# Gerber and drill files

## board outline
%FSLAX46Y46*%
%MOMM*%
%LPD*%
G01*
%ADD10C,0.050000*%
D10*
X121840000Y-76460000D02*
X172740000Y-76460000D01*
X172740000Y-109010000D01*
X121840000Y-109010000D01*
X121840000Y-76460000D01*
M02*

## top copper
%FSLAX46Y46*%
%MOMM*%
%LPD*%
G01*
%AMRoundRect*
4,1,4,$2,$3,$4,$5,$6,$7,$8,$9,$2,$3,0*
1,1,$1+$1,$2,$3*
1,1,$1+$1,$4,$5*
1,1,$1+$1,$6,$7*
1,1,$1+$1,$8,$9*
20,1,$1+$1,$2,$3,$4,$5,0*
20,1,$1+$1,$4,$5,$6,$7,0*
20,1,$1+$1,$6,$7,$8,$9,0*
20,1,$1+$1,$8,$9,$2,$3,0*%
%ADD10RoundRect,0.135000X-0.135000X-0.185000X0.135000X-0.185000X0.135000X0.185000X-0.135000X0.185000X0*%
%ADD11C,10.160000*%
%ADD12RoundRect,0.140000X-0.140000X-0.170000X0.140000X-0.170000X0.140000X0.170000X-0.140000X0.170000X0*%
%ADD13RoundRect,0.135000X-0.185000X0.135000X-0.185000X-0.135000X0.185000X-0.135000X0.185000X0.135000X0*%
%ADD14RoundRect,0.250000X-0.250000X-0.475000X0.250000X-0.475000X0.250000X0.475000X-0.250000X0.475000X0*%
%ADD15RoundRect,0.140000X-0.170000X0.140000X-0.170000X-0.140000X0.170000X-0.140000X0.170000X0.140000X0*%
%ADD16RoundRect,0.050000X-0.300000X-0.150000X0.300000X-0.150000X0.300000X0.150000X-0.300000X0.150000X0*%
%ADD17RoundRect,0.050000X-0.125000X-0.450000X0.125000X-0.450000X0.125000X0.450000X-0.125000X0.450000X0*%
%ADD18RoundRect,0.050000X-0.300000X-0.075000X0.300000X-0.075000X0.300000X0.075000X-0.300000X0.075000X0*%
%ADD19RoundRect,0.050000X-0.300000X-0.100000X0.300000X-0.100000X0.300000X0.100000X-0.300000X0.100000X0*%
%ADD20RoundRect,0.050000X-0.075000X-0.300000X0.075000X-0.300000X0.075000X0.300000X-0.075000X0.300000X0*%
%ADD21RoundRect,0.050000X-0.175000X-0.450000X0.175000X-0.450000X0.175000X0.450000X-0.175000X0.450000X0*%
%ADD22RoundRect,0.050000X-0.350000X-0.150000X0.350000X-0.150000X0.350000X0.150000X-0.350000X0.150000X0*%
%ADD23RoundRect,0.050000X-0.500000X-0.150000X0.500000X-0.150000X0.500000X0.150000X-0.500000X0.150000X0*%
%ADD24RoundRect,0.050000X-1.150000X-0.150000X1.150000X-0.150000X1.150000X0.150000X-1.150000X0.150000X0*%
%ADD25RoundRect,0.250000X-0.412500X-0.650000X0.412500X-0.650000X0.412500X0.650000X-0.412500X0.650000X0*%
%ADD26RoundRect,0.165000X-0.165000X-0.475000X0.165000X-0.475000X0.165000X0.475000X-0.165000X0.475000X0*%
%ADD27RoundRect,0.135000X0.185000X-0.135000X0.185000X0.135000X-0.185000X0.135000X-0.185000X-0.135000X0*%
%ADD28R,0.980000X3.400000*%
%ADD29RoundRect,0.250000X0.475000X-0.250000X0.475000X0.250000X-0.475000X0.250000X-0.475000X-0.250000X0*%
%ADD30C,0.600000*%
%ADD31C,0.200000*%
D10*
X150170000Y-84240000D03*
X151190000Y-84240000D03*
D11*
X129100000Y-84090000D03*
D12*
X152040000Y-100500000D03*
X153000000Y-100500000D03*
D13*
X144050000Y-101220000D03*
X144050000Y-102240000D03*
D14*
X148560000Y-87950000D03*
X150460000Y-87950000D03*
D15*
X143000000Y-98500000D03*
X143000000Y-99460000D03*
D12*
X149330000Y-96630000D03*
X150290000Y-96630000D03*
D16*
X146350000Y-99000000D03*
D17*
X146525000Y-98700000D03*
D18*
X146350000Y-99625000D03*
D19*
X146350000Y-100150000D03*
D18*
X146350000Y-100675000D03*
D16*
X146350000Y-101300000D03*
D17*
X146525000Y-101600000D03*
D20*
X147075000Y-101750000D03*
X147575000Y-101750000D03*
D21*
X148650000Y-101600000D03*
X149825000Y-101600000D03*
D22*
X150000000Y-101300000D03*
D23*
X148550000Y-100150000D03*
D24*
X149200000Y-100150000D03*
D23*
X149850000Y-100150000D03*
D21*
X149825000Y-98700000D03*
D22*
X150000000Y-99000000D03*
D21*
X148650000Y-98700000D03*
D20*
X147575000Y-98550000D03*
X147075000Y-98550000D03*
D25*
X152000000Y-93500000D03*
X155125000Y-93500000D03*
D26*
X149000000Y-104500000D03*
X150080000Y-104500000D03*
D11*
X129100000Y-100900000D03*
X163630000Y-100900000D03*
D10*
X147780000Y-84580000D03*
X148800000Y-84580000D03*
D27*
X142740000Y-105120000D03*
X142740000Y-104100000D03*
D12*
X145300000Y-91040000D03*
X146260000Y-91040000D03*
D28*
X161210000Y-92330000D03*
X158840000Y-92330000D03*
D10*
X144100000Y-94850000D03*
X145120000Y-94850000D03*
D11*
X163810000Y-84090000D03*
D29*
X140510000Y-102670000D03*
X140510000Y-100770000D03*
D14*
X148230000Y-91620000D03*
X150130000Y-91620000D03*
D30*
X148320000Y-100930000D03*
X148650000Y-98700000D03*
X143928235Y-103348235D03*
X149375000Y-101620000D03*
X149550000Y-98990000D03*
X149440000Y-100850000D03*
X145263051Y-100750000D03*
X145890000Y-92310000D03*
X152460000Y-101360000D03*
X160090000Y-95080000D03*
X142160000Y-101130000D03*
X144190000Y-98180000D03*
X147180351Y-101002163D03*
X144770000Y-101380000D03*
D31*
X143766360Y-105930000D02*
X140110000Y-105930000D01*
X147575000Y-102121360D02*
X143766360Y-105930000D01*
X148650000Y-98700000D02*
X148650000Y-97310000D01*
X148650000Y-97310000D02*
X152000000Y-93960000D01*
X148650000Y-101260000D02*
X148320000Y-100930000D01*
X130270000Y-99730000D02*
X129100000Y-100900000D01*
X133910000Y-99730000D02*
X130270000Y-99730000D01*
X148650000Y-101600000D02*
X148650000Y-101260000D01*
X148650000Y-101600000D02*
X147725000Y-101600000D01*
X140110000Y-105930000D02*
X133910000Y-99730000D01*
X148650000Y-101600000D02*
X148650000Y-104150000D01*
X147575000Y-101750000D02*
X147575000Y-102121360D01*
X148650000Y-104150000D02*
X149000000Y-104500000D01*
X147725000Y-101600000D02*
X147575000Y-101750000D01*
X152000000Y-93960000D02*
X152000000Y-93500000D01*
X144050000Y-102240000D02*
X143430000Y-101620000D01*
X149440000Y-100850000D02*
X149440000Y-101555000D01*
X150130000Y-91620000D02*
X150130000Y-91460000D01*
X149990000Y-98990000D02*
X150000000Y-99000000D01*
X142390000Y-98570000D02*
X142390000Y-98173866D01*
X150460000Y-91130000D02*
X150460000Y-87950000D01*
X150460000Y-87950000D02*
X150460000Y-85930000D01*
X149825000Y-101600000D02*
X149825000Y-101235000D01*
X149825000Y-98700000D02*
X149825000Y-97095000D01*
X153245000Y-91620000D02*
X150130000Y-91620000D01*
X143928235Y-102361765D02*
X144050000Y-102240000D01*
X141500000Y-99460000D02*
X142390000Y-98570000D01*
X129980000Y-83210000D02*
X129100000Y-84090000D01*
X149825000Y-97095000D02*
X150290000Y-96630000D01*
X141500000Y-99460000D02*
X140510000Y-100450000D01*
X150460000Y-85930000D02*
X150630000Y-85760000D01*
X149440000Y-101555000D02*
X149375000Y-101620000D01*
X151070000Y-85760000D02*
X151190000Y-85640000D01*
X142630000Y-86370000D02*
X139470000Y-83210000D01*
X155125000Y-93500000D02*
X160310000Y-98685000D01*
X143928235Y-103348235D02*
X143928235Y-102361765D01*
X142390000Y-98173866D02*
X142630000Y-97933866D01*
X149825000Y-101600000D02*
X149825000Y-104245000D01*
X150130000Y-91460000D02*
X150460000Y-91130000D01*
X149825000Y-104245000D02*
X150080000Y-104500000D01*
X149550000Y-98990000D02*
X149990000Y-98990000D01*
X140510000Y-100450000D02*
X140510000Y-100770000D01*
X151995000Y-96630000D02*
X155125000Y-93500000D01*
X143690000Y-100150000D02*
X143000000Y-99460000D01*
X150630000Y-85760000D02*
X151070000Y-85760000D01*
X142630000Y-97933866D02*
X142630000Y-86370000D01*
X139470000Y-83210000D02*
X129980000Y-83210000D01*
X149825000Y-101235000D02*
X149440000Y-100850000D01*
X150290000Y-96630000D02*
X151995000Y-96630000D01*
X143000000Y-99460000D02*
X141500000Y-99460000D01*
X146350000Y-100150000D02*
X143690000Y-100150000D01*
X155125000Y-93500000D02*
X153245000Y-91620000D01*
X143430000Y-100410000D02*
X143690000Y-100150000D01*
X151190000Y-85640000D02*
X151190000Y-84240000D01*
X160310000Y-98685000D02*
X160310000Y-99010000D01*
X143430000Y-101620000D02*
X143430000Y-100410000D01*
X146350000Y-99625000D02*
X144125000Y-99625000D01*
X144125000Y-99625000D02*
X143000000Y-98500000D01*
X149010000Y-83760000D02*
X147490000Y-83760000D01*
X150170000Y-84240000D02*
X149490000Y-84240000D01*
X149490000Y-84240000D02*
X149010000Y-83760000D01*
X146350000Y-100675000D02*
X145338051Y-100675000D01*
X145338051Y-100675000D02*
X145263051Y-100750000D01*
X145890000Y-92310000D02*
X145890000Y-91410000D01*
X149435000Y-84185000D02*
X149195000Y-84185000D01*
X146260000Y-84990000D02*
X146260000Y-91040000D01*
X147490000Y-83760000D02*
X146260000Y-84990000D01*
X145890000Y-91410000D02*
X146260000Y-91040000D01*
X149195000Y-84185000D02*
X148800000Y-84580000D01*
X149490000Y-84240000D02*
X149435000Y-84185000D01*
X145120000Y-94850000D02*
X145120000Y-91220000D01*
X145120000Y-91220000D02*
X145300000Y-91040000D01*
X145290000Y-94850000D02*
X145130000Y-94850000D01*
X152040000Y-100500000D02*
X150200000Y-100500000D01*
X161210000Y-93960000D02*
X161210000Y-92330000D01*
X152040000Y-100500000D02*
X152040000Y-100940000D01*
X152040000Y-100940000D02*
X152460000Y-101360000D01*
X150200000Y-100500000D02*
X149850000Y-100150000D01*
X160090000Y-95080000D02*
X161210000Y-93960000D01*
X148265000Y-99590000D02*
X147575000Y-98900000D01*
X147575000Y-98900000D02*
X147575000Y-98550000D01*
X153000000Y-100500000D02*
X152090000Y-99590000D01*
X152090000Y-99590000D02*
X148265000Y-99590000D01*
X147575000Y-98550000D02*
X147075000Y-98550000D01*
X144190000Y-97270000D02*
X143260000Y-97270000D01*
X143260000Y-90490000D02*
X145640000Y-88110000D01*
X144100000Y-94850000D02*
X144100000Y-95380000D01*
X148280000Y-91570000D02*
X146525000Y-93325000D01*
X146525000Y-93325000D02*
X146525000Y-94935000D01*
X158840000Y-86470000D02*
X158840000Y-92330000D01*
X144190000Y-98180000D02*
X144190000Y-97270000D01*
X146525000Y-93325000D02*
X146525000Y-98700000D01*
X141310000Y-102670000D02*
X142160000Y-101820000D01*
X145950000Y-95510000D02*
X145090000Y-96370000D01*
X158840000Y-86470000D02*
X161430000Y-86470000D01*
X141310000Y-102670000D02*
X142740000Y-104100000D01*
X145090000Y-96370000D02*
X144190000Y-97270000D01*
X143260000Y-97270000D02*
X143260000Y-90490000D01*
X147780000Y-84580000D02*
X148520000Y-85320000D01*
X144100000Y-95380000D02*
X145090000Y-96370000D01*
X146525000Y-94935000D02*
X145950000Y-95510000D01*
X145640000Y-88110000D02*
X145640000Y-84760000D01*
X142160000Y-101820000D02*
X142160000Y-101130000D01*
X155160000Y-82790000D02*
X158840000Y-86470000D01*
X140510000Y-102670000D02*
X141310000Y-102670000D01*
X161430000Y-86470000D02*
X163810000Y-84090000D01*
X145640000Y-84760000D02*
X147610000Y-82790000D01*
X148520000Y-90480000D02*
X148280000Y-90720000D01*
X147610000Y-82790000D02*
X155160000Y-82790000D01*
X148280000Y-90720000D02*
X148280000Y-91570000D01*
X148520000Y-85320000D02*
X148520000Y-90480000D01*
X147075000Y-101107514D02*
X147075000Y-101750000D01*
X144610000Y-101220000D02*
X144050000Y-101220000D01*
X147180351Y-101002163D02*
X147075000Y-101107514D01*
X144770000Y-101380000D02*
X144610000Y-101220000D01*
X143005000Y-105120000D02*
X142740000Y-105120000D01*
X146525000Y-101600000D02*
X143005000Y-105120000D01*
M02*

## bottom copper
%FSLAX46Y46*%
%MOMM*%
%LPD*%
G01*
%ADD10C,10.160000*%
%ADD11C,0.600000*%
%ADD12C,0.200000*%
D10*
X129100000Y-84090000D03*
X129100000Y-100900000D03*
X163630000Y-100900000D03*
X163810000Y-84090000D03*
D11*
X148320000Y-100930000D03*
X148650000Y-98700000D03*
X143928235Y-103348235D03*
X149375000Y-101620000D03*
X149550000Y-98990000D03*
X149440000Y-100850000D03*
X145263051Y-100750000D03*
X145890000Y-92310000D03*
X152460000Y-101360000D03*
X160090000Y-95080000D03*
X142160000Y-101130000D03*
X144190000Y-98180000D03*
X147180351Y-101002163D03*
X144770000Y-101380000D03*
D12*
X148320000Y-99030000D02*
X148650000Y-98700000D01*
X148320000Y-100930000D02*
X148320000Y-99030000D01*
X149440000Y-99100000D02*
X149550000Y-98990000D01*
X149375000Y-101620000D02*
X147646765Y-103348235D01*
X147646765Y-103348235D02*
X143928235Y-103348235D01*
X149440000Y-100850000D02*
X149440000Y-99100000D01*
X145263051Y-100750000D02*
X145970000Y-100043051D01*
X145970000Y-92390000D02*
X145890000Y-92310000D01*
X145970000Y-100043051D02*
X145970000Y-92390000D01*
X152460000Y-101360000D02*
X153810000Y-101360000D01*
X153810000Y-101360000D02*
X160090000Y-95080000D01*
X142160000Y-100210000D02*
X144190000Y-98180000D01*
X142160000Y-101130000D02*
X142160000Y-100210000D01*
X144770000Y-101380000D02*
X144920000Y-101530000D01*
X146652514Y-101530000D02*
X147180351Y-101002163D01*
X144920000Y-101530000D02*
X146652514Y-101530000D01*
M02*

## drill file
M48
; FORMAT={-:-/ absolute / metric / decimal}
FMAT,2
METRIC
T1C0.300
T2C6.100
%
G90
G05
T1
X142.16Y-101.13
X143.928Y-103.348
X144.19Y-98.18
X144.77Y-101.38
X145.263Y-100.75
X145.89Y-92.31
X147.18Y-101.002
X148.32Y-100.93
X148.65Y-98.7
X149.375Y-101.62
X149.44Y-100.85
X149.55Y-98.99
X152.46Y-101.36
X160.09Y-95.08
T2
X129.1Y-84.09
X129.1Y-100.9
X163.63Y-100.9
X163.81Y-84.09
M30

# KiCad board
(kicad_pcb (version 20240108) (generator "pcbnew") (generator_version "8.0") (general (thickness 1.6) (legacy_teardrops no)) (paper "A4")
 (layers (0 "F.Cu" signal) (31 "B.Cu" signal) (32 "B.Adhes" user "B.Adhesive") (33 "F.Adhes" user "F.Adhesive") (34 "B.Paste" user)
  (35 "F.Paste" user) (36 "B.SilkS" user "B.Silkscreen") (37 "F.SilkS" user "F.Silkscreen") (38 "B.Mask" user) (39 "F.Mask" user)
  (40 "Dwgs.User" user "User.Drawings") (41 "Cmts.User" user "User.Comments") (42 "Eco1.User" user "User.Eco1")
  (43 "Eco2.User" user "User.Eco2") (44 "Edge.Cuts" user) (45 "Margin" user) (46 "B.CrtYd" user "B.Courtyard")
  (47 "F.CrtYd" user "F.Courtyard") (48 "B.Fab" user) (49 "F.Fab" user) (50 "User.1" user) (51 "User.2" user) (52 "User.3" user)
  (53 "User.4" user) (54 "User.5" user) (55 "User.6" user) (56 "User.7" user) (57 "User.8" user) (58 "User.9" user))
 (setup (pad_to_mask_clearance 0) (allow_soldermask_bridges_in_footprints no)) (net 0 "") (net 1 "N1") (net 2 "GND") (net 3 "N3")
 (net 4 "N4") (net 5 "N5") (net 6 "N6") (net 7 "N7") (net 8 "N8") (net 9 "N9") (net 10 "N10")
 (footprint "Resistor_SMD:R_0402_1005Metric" (layer "F.Cu") (at 150.68 84.24)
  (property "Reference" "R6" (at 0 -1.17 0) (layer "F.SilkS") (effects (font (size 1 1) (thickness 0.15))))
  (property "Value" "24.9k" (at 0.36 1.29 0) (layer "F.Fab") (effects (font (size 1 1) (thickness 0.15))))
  (pad "1" smd roundrect (at -0.51 0) (size 0.54 0.64) (layers "F.Cu" "F.Paste" "F.Mask") (roundrect_rratio 0.25) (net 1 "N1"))
  (pad "2" smd roundrect (at 0.51 0) (size 0.54 0.64) (layers "F.Cu" "F.Paste" "F.Mask") (roundrect_rratio 0.25) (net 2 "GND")))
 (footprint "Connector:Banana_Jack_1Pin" (layer "F.Cu") (at 129.1 84.09)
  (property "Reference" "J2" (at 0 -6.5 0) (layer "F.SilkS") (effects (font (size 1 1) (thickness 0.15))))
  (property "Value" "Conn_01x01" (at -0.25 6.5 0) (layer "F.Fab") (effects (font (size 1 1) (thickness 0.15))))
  (pad "1" thru_hole circle (at 0 0) (size 10.16 10.16) (drill 6.1) (layers "*.Cu" "*.Mask") (remove_unused_layers no) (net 2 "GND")))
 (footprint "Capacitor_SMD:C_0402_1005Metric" (layer "F.Cu") (at 152.52 100.5)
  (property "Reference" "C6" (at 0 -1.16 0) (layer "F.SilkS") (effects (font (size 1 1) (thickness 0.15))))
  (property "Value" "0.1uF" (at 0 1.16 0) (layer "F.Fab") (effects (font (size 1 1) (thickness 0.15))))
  (pad "1" smd roundrect (at -0.48 0) (size 0.56 0.62) (layers "F.Cu" "F.Paste" "F.Mask") (roundrect_rratio 0.25) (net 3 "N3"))
  (pad "2" smd roundrect (at 0.48 0) (size 0.56 0.62) (layers "F.Cu" "F.Paste" "F.Mask") (roundrect_rratio 0.25) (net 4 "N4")))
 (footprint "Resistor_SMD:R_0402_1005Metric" (layer "F.Cu") (at 144.05 101.73 -90)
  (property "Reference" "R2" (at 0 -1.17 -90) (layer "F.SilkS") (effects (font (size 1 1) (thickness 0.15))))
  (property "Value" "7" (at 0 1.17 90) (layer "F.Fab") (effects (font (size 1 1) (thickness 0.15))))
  (pad "1" smd roundrect (at -0.51 0 270) (size 0.54 0.64) (layers "F.Cu" "F.Paste" "F.Mask") (roundrect_rratio 0.25) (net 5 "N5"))
  (pad "2" smd roundrect (at 0.51 0 270) (size 0.54 0.64) (layers "F.Cu" "F.Paste" "F.Mask") (roundrect_rratio 0.25) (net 2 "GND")))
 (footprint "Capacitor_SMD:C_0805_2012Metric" (layer "F.Cu") (at 149.51 87.95)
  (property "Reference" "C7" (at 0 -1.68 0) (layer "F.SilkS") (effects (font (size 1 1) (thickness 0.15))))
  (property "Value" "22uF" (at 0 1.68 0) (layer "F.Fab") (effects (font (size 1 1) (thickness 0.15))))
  (pad "1" smd roundrect (at -0.95 0) (size 1 1.45) (layers "F.Cu" "F.Paste" "F.Mask") (roundrect_rratio 0.25) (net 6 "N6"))
  (pad "2" smd roundrect (at 0.95 0) (size 1 1.45) (layers "F.Cu" "F.Paste" "F.Mask") (roundrect_rratio 0.25) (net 2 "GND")))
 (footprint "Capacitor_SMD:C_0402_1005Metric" (layer "F.Cu") (at 143 98.98 -90)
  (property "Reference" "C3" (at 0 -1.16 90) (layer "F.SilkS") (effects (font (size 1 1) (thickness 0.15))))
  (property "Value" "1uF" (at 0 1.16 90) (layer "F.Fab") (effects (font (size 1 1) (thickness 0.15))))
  (pad "1" smd roundrect (at -0.48 0 270) (size 0.56 0.62) (layers "F.Cu" "F.Paste" "F.Mask") (roundrect_rratio 0.25) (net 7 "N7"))
  (pad "2" smd roundrect (at 0.48 0 270) (size 0.56 0.62) (layers "F.Cu" "F.Paste" "F.Mask") (roundrect_rratio 0.25) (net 2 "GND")))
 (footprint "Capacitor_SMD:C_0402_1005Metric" (layer "F.Cu") (at 149.81 96.63)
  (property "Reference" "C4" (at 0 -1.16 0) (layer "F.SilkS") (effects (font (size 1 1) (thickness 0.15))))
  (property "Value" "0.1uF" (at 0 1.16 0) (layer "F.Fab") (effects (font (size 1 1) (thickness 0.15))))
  (pad "1" smd roundrect (at -0.48 0) (size 0.56 0.62) (layers "F.Cu" "F.Paste" "F.Mask") (roundrect_rratio 0.25) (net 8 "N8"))
  (pad "2" smd roundrect (at 0.48 0) (size 0.56 0.62) (layers "F.Cu" "F.Paste" "F.Mask") (roundrect_rratio 0.25) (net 2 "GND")))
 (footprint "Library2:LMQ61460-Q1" (layer "F.Cu") (at 148.2 100.15)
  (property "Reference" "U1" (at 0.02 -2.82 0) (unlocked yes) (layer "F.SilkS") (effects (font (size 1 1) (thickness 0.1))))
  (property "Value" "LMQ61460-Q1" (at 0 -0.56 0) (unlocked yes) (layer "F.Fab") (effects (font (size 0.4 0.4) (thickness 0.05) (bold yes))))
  (pad "1" smd roundrect (at -1.85 -1.15) (size 0.7 0.4) (layers "F.Cu" "F.Paste" "F.Mask") (roundrect_rratio 0.125) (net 6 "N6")
   (solder_paste_margin_ratio -0.05) (thermal_bridge_angle 45))
  (pad "1" smd roundrect (at -1.675 -1.45) (size 0.35 1) (layers "F.Cu" "F.Paste" "F.Mask") (roundrect_rratio 0.1428571429) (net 6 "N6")
   (solder_paste_margin_ratio -0.05) (thermal_bridge_angle 45))
  (pad "2" smd roundrect (at -1.85 -0.525) (size 0.7 0.25) (layers "F.Cu" "F.Paste" "F.Mask") (roundrect_rratio 0.2) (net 7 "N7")
   (thermal_bridge_angle 45))
  (pad "3" smd roundrect (at -1.85 0) (size 0.7 0.3) (layers "F.Cu" "F.Paste" "F.Mask") (roundrect_rratio 0.1666666667) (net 2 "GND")
   (thermal_bridge_angle 45))
  (pad "4" smd roundrect (at -1.85 0.525) (size 0.7 0.25) (layers "F.Cu" "F.Paste" "F.Mask") (roundrect_rratio 0.2) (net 1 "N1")
   (thermal_bridge_angle 45))
  (pad "5" smd roundrect (at -1.85 1.15) (size 0.7 0.4) (layers "F.Cu" "F.Paste" "F.Mask") (roundrect_rratio 0.125) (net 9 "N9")
   (solder_paste_margin_ratio -0.05) (thermal_bridge_angle 45))
  (pad "5" smd roundrect (at -1.675 1.45) (size 0.35 1) (layers "F.Cu" "F.Paste" "F.Mask") (roundrect_rratio 0.1428571429) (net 9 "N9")
   (solder_paste_margin_ratio -0.05) (thermal_bridge_angle 45))
  (pad "6" smd roundrect (at -1.125 1.6) (size 0.25 0.7) (layers "F.Cu" "F.Paste" "F.Mask") (roundrect_rratio 0.2) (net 5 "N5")
   (thermal_bridge_angle 45))
  (pad "7" smd roundrect (at -0.625 1.6) (size 0.25 0.7) (layers "F.Cu" "F.Paste" "F.Mask") (roundrect_rratio 0.2) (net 8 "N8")
   (thermal_bridge_angle 45))
  (pad "8" smd roundrect (at 0.45 1.45) (size 0.45 1) (layers "F.Cu" "F.Paste" "F.Mask") (roundrect_rratio 0.1111111111) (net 8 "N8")
   (thermal_bridge_angle 45))
  (pad "9" smd roundrect (at 1.625 1.45) (size 0.45 1) (layers "F.Cu" "F.Paste" "F.Mask") (roundrect_rratio 0.1111111111) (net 2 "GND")
   (solder_paste_margin_ratio -0.05) (thermal_bridge_angle 45))
  (pad "9" smd roundrect (at 1.8 1.15) (size 0.8 0.4) (layers "F.Cu" "F.Paste" "F.Mask") (roundrect_rratio 0.125) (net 2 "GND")
   (solder_paste_margin_ratio -0.05) (thermal_bridge_angle 45))
  (pad "10" smd roundrect (at 0.35 0) (size 1.1 0.4) (layers "F.Cu" "F.Paste" "F.Mask") (roundrect_rratio 0.125) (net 3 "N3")
   (thermal_bridge_angle 45))
  (pad "10" smd roundrect (at 1 0) (size 2.4 0.4) (layers "F.Cu" "F.Paste" "F.Mask") (roundrect_rratio 0.125) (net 3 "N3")
   (thermal_bridge_angle 45))
  (pad "10" smd roundrect (at 1.65 0) (size 1.1 0.4) (layers "F.Cu" "F.Paste" "F.Mask") (roundrect_rratio 0.125) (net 3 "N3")
   (thermal_bridge_angle 45))
  (pad "11" smd roundrect (at 1.625 -1.45) (size 0.45 1) (layers "F.Cu" "F.Paste" "F.Mask") (roundrect_rratio 0.1111111111) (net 2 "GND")
   (solder_paste_margin_ratio -0.05) (thermal_bridge_angle 45))
  (pad "11" smd roundrect (at 1.8 -1.15) (size 0.8 0.4) (layers "F.Cu" "F.Paste" "F.Mask") (roundrect_rratio 0.125) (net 2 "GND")
   (solder_paste_margin_ratio -0.05) (thermal_bridge_angle 45))
  (pad "12" smd roundrect (at 0.45 -1.45) (size 0.45 1) (layers "F.Cu" "F.Paste" "F.Mask") (roundrect_rratio 0.1111111111) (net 8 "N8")
   (thermal_bridge_angle 45))
  (pad "13" smd roundrect (at -0.625 -1.6) (size 0.25 0.7) (layers "F.Cu" "F.Paste" "F.Mask") (roundrect_rratio 0.2) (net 4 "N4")
   (thermal_bridge_angle 45))
  (pad "14" smd roundrect (at -1.125 -1.6) (size 0.25 0.7) (layers "F.Cu" "F.Paste" "F.Mask") (roundrect_rratio 0.2) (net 4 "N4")
   (thermal_bridge_angle 45)))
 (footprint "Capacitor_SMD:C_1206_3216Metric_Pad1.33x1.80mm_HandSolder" (layer "F.Cu") (at 153.5625 93.5)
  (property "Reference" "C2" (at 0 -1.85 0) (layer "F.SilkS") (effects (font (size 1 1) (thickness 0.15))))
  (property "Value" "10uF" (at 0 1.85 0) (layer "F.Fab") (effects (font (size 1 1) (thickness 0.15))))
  (pad "1" smd roundrect (at -1.5625 0) (size 1.325 1.8) (layers "F.Cu" "F.Paste" "F.Mask") (roundrect_rratio 0.188679) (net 8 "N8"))
  (pad "2" smd roundrect (at 1.5625 0) (size 1.325 1.8) (layers "F.Cu" "F.Paste" "F.Mask") (roundrect_rratio 0.188679) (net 2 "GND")))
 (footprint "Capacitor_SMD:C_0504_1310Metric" (layer "F.Cu") (at 149.54 104.5)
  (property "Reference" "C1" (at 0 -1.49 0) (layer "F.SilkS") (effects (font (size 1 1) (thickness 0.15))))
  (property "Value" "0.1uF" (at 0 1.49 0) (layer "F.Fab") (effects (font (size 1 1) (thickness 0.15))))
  (pad "1" smd roundrect (at -0.54 0) (size 0.66 1.28) (layers "F.Cu" "F.Paste" "F.Mask") (roundrect_rratio 0.25) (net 8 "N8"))
  (pad "2" smd roundrect (at 0.54 0) (size 0.66 1.28) (layers "F.Cu" "F.Paste" "F.Mask") (roundrect_rratio 0.25) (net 2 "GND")))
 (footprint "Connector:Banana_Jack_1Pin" (layer "F.Cu") (at 129.1 100.9)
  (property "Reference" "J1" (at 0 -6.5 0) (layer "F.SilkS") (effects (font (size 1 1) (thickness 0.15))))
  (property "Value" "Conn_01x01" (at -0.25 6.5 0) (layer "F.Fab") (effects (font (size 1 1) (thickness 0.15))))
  (pad "1" thru_hole circle (at 0 0) (size 10.16 10.16) (drill 6.1) (layers "*.Cu" "*.Mask") (remove_unused_layers no) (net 8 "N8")))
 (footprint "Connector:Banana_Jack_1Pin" (layer "F.Cu") (at 163.63 100.9)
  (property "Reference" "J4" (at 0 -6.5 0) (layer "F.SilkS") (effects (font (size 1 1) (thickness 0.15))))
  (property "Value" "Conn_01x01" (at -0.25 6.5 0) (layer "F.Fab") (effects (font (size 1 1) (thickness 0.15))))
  (pad "1" thru_hole circle (at 0 0) (size 10.16 10.16) (drill 6.1) (layers "*.Cu" "*.Mask") (remove_unused_layers no) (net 2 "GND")))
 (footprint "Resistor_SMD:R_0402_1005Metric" (layer "F.Cu") (at 148.29 84.58)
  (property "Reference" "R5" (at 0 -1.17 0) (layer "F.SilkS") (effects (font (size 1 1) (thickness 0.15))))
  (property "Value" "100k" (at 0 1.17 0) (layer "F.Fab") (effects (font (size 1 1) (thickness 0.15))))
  (pad "1" smd roundrect (at -0.51 0) (size 0.54 0.64) (layers "F.Cu" "F.Paste" "F.Mask") (roundrect_rratio 0.25) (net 6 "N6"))
  (pad "2" smd roundrect (at 0.51 0) (size 0.54 0.64) (layers "F.Cu" "F.Paste" "F.Mask") (roundrect_rratio 0.25) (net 1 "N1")))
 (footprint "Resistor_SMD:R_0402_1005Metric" (layer "F.Cu") (at 142.74 104.61 90)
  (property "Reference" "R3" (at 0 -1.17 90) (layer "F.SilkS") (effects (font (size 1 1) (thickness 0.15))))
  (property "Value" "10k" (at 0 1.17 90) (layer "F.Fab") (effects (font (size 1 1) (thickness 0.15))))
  (pad "1" smd roundrect (at -0.51 0 90) (size 0.54 0.64) (layers "F.Cu" "F.Paste" "F.Mask") (roundrect_rratio 0.25) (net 9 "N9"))
  (pad "2" smd roundrect (at 0.51 0 90) (size 0.54 0.64) (layers "F.Cu" "F.Paste" "F.Mask") (roundrect_rratio 0.25) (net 6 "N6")))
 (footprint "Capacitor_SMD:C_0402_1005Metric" (layer "F.Cu") (at 145.78 91.04)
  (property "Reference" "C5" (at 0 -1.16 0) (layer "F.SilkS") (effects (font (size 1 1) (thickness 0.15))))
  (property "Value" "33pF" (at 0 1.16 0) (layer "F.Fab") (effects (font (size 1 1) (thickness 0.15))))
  (pad "1" smd roundrect (at -0.48 0) (size 0.56 0.62) (layers "F.Cu" "F.Paste" "F.Mask") (roundrect_rratio 0.25) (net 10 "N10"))
  (pad "2" smd roundrect (at 0.48 0) (size 0.56 0.62) (layers "F.Cu" "F.Paste" "F.Mask") (roundrect_rratio 0.25) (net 1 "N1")))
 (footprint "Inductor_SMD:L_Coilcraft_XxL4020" (layer "F.Cu") (at 160.025 92.33 180)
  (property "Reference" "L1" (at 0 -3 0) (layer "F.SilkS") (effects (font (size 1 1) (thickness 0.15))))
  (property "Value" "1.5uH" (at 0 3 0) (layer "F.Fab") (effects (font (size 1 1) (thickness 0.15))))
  (pad "1" smd rect (at -1.185 0 180) (size 0.98 3.4) (layers "F.Cu" "F.Paste" "F.Mask") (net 3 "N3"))
  (pad "2" smd rect (at 1.185 0 180) (size 0.98 3.4) (layers "F.Cu" "F.Paste" "F.Mask") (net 6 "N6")))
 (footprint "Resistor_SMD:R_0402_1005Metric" (layer "F.Cu") (at 144.61 94.85)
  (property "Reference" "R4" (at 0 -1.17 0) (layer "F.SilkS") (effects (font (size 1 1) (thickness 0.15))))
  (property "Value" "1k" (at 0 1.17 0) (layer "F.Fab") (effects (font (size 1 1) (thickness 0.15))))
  (pad "1" smd roundrect (at -0.51 0) (size 0.54 0.64) (layers "F.Cu" "F.Paste" "F.Mask") (roundrect_rratio 0.25) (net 6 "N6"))
  (pad "2" smd roundrect (at 0.51 0) (size 0.54 0.64) (layers "F.Cu" "F.Paste" "F.Mask") (roundrect_rratio 0.25) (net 10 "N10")))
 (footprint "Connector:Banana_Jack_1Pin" (layer "F.Cu") (at 163.81 84.09)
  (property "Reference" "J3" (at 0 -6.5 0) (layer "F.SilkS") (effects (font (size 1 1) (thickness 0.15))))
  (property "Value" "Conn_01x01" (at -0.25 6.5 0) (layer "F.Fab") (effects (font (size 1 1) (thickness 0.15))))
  (pad "1" thru_hole circle (at 0 0) (size 10.16 10.16) (drill 6.1) (layers "*.Cu" "*.Mask") (remove_unused_layers no) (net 6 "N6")))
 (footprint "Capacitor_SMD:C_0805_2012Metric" (layer "F.Cu") (at 140.51 101.72 90)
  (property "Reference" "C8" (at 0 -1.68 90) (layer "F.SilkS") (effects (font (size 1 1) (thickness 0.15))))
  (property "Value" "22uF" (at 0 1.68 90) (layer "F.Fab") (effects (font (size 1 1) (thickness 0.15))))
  (pad "1" smd roundrect (at -0.95 0 90) (size 1 1.45) (layers "F.Cu" "F.Paste" "F.Mask") (roundrect_rratio 0.25) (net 6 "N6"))
  (pad "2" smd roundrect (at 0.95 0 90) (size 1 1.45) (layers "F.Cu" "F.Paste" "F.Mask") (roundrect_rratio 0.25) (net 2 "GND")))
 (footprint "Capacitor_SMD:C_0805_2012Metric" (layer "F.Cu") (at 149.18 91.62)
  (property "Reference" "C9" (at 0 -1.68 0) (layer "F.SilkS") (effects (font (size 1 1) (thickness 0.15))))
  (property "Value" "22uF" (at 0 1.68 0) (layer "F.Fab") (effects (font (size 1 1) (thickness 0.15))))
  (pad "1" smd roundrect (at -0.95 0) (size 1 1.45) (layers "F.Cu" "F.Paste" "F.Mask") (roundrect_rratio 0.25) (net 6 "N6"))
  (pad "2" smd roundrect (at 0.95 0) (size 1 1.45) (layers "F.Cu" "F.Paste" "F.Mask") (roundrect_rratio 0.25) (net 2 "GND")))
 (gr_rect (start 121.84 76.46) (end 172.74 109.01) (stroke (width 0.05) (type default)) (fill none) (layer "Edge.Cuts"))
 (segment (start 143.76636 105.93) (end 140.11 105.93) (width 0.2) (layer "F.Cu") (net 8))
 (segment (start 147.575 102.12136) (end 143.76636 105.93) (width 0.2) (layer "F.Cu") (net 8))
 (segment (start 148.65 98.7) (end 148.65 97.31) (width 0.2) (layer "F.Cu") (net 8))
 (segment (start 148.65 97.31) (end 152 93.96) (width 0.2) (layer "F.Cu") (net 8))
 (segment (start 148.65 101.26) (end 148.32 100.93) (width 0.2) (layer "F.Cu") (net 8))
 (segment (start 130.27 99.73) (end 129.1 100.9) (width 0.2) (layer "F.Cu") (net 8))
 (segment (start 133.91 99.73) (end 130.27 99.73) (width 0.2) (layer "F.Cu") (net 8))
 (segment (start 148.65 101.6) (end 148.65 101.26) (width 0.2) (layer "F.Cu") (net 8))
 (segment (start 148.65 101.6) (end 147.725 101.6) (width 0.2) (layer "F.Cu") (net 8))
 (segment (start 140.11 105.93) (end 133.91 99.73) (width 0.2) (layer "F.Cu") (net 8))
 (segment (start 148.65 101.6) (end 148.65 104.15) (width 0.2) (layer "F.Cu") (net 8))
 (segment (start 147.575 101.75) (end 147.575 102.12136) (width 0.2) (layer "F.Cu") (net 8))
 (segment (start 148.65 104.15) (end 149 104.5) (width 0.2) (layer "F.Cu") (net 8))
 (segment (start 147.725 101.6) (end 147.575 101.75) (width 0.2) (layer "F.Cu") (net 8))
 (segment (start 152 93.96) (end 152 93.5) (width 0.2) (layer "F.Cu") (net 8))
 (via (at 148.32 100.93) (size 0.6) (drill 0.3) (layers "F.Cu" "B.Cu") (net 8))
 (via (at 148.65 98.7) (size 0.6) (drill 0.3) (layers "F.Cu" "B.Cu") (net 8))
 (segment (start 148.32 99.03) (end 148.65 98.7) (width 0.2) (layer "B.Cu") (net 8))
 (segment (start 148.32 100.93) (end 148.32 99.03) (width 0.2) (layer "B.Cu") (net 8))
 (segment (start 144.05 102.24) (end 143.43 101.62) (width 0.2) (layer "F.Cu") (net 2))
 (segment (start 149.44 100.85) (end 149.44 101.555) (width 0.2) (layer "F.Cu") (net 2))
 (segment (start 150.13 91.62) (end 150.13 91.46) (width 0.2) (layer "F.Cu") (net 2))
 (segment (start 149.99 98.99) (end 150 99) (width 0.2) (layer "F.Cu") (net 2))
 (segment (start 142.39 98.57) (end 142.39 98.173866) (width 0.2) (layer "F.Cu") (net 2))
 (segment (start 150.46 91.13) (end 150.46 87.95) (width 0.2) (layer "F.Cu") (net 2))
 (segment (start 150.46 87.95) (end 150.46 85.93) (width 0.2) (layer "F.Cu") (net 2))
 (segment (start 149.825 101.6) (end 149.825 101.235) (width 0.2) (layer "F.Cu") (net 2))
 (segment (start 149.825 98.7) (end 149.825 97.095) (width 0.2) (layer "F.Cu") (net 2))
 (segment (start 153.245 91.62) (end 150.13 91.62) (width 0.2) (layer "F.Cu") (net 2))
 (segment (start 143.928235 102.361765) (end 144.05 102.24) (width 0.2) (layer "F.Cu") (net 2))
 (segment (start 141.5 99.46) (end 142.39 98.57) (width 0.2) (layer "F.Cu") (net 2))
 (segment (start 129.98 83.21) (end 129.1 84.09) (width 0.2) (layer "F.Cu") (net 2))
 (segment (start 149.825 97.095) (end 150.29 96.63) (width 0.2) (layer "F.Cu") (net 2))
 (segment (start 141.5 99.46) (end 140.51 100.45) (width 0.2) (layer "F.Cu") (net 2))
 (segment (start 150.46 85.93) (end 150.63 85.76) (width 0.2) (layer "F.Cu") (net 2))
 (segment (start 149.44 101.555) (end 149.375 101.62) (width 0.2) (layer "F.Cu") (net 2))
 (segment (start 151.07 85.76) (end 151.19 85.64) (width 0.2) (layer "F.Cu") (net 2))
 (segment (start 142.63 86.37) (end 139.47 83.21) (width 0.2) (layer "F.Cu") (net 2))
 (segment (start 155.125 93.5) (end 160.31 98.685) (width 0.2) (layer "F.Cu") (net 2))
 (segment (start 143.928235 103.348235) (end 143.928235 102.361765) (width 0.2) (layer "F.Cu") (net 2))
 (segment (start 142.39 98.173866) (end 142.63 97.933866) (width 0.2) (layer "F.Cu") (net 2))
 (segment (start 149.825 101.6) (end 149.825 104.245) (width 0.2) (layer "F.Cu") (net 2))
 (segment (start 150.13 91.46) (end 150.46 91.13) (width 0.2) (layer "F.Cu") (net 2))
 (segment (start 149.825 104.245) (end 150.08 104.5) (width 0.2) (layer "F.Cu") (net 2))
 (segment (start 149.55 98.99) (end 149.99 98.99) (width 0.2) (layer "F.Cu") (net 2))
 (segment (start 140.51 100.45) (end 140.51 100.77) (width 0.2) (layer "F.Cu") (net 2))
 (segment (start 151.995 96.63) (end 155.125 93.5) (width 0.2) (layer "F.Cu") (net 2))
 (segment (start 143.69 100.15) (end 143 99.46) (width 0.2) (layer "F.Cu") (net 2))
 (segment (start 150.63 85.76) (end 151.07 85.76) (width 0.2) (layer "F.Cu") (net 2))
 (segment (start 142.63 97.933866) (end 142.63 86.37) (width 0.2) (layer "F.Cu") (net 2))
 (segment (start 139.47 83.21) (end 129.98 83.21) (width 0.2) (layer "F.Cu") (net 2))
 (segment (start 149.825 101.235) (end 149.44 100.85) (width 0.2) (layer "F.Cu") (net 2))
 (segment (start 150.29 96.63) (end 151.995 96.63) (width 0.2) (layer "F.Cu") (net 2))
 (segment (start 143 99.46) (end 141.5 99.46) (width 0.2) (layer "F.Cu") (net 2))
 (segment (start 146.35 100.15) (end 143.69 100.15) (width 0.2) (layer "F.Cu") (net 2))
 (segment (start 155.125 93.5) (end 153.245 91.62) (width 0.2) (layer "F.Cu") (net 2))
 (segment (start 143.43 100.41) (end 143.69 100.15) (width 0.2) (layer "F.Cu") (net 2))
 (segment (start 151.19 85.64) (end 151.19 84.24) (width 0.2) (layer "F.Cu") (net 2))
 (segment (start 160.31 98.685) (end 160.31 99.01) (width 0.2) (layer "F.Cu") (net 2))
 (segment (start 143.43 101.62) (end 143.43 100.41) (width 0.2) (layer "F.Cu") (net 2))
 (via (at 143.928235 103.348235) (size 0.6) (drill 0.3) (layers "F.Cu" "B.Cu") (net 2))
 (via (at 149.375 101.62) (size 0.6) (drill 0.3) (layers "F.Cu" "B.Cu") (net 2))
 (via (at 149.55 98.99) (size 0.6) (drill 0.3) (layers "F.Cu" "B.Cu") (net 2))
 (via (at 149.44 100.85) (size 0.6) (drill 0.3) (layers "F.Cu" "B.Cu") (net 2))
 (segment (start 149.44 99.1) (end 149.55 98.99) (width 0.2) (layer "B.Cu") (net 2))
 (segment (start 149.375 101.62) (end 147.646765 103.348235) (width 0.2) (layer "B.Cu") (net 2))
 (segment (start 147.646765 103.348235) (end 143.928235 103.348235) (width 0.2) (layer "B.Cu") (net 2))
 (segment (start 149.44 100.85) (end 149.44 99.1) (width 0.2) (layer "B.Cu") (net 2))
 (segment (start 146.35 99.625) (end 144.125 99.625) (width 0.2) (layer "F.Cu") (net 7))
 (segment (start 144.125 99.625) (end 143 98.5) (width 0.2) (layer "F.Cu") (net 7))
 (segment (start 149.01 83.76) (end 147.49 83.76) (width 0.2) (layer "F.Cu") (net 1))
 (segment (start 150.17 84.24) (end 149.49 84.24) (width 0.2) (layer "F.Cu") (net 1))
 (segment (start 149.49 84.24) (end 149.01 83.76) (width 0.2) (layer "F.Cu") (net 1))
 (segment (start 146.35 100.675) (end 145.338051 100.675) (width 0.2) (layer "F.Cu") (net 1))
 (segment (start 145.338051 100.675) (end 145.263051 100.75) (width 0.2) (layer "F.Cu") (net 1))
 (segment (start 145.89 92.31) (end 145.89 91.41) (width 0.2) (layer "F.Cu") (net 1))
 (segment (start 149.435 84.185) (end 149.195 84.185) (width 0.2) (layer "F.Cu") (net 1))
 (segment (start 146.26 84.99) (end 146.26 91.04) (width 0.2) (layer "F.Cu") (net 1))
 (segment (start 147.49 83.76) (end 146.26 84.99) (width 0.2) (layer "F.Cu") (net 1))
 (segment (start 145.89 91.41) (end 146.26 91.04) (width 0.2) (layer "F.Cu") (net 1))
 (segment (start 149.195 84.185) (end 148.8 84.58) (width 0.2) (layer "F.Cu") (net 1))
 (segment (start 149.49 84.24) (end 149.435 84.185) (width 0.2) (layer "F.Cu") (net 1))
 (via (at 145.263051 100.75) (size 0.6) (drill 0.3) (layers "F.Cu" "B.Cu") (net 1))
 (via (at 145.89 92.31) (size 0.6) (drill 0.3) (layers "F.Cu" "B.Cu") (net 1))
 (segment (start 145.263051 100.75) (end 145.97 100.043051) (width 0.2) (layer "B.Cu") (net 1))
 (segment (start 145.97 92.39) (end 145.89 92.31) (width 0.2) (layer "B.Cu") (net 1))
 (segment (start 145.97 100.043051) (end 145.97 92.39) (width 0.2) (layer "B.Cu") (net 1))
 (segment (start 145.12 94.85) (end 145.12 91.22) (width 0.2) (layer "F.Cu") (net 10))
 (segment (start 145.12 91.22) (end 145.3 91.04) (width 0.2) (layer "F.Cu") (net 10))
 (segment (start 145.29 94.85) (end 145.13 94.85) (width 0.2) (layer "F.Cu") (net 10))
 (segment (start 152.04 100.5) (end 150.2 100.5) (width 0.2) (layer "F.Cu") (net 3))
 (segment (start 161.21 93.96) (end 161.21 92.33) (width 0.2) (layer "F.Cu") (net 3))
 (segment (start 152.04 100.5) (end 152.04 100.94) (width 0.2) (layer "F.Cu") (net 3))
 (segment (start 152.04 100.94) (end 152.46 101.36) (width 0.2) (layer "F.Cu") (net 3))
 (segment (start 150.2 100.5) (end 149.85 100.15) (width 0.2) (layer "F.Cu") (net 3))
 (segment (start 160.09 95.08) (end 161.21 93.96) (width 0.2) (layer "F.Cu") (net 3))
 (via (at 152.46 101.36) (size 0.6) (drill 0.3) (layers "F.Cu" "B.Cu") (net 3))
 (via (at 160.09 95.08) (size 0.6) (drill 0.3) (layers "F.Cu" "B.Cu") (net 3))
 (segment (start 152.46 101.36) (end 153.81 101.36) (width 0.2) (layer "B.Cu") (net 3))
 (segment (start 153.81 101.36) (end 160.09 95.08) (width 0.2) (layer "B.Cu") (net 3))
 (segment (start 148.265 99.59) (end 147.575 98.9) (width 0.2) (layer "F.Cu") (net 4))
 (segment (start 147.575 98.9) (end 147.575 98.55) (width 0.2) (layer "F.Cu") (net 4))
 (segment (start 153 100.5) (end 152.09 99.59) (width 0.2) (layer "F.Cu") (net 4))
 (segment (start 152.09 99.59) (end 148.265 99.59) (width 0.2) (layer "F.Cu") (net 4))
 (segment (start 147.575 98.55) (end 147.075 98.55) (width 0.2) (layer "F.Cu") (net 4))
 (segment (start 144.19 97.27) (end 143.26 97.27) (width 0.2) (layer "F.Cu") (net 6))
 (segment (start 143.26 90.49) (end 145.64 88.11) (width 0.2) (layer "F.Cu") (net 6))
 (segment (start 144.1 94.85) (end 144.1 95.38) (width 0.2) (layer "F.Cu") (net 6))
 (segment (start 148.28 91.57) (end 146.525 93.325) (width 0.2) (layer "F.Cu") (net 6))
 (segment (start 146.525 93.325) (end 146.525 94.935) (width 0.2) (layer "F.Cu") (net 6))
 (segment (start 158.84 86.47) (end 158.84 92.33) (width 0.2) (layer "F.Cu") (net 6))
 (segment (start 144.19 98.18) (end 144.19 97.27) (width 0.2) (layer "F.Cu") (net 6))
 (segment (start 146.525 93.325) (end 146.525 98.7) (width 0.2) (layer "F.Cu") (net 6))
 (segment (start 141.31 102.67) (end 142.16 101.82) (width 0.2) (layer "F.Cu") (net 6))
 (segment (start 145.95 95.51) (end 145.09 96.37) (width 0.2) (layer "F.Cu") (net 6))
 (segment (start 158.84 86.47) (end 161.43 86.47) (width 0.2) (layer "F.Cu") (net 6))
 (segment (start 141.31 102.67) (end 142.74 104.1) (width 0.2) (layer "F.Cu") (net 6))
 (segment (start 145.09 96.37) (end 144.19 97.27) (width 0.2) (layer "F.Cu") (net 6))
 (segment (start 143.26 97.27) (end 143.26 90.49) (width 0.2) (layer "F.Cu") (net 6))
 (segment (start 147.78 84.58) (end 148.52 85.32) (width 0.2) (layer "F.Cu") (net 6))
 (segment (start 144.1 95.38) (end 145.09 96.37) (width 0.2) (layer "F.Cu") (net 6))
 (segment (start 146.525 94.935) (end 145.95 95.51) (width 0.2) (layer "F.Cu") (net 6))
 (segment (start 145.64 88.11) (end 145.64 84.76) (width 0.2) (layer "F.Cu") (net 6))
 (segment (start 142.16 101.82) (end 142.16 101.13) (width 0.2) (layer "F.Cu") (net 6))
 (segment (start 155.16 82.79) (end 158.84 86.47) (width 0.2) (layer "F.Cu") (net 6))
 (segment (start 140.51 102.67) (end 141.31 102.67) (width 0.2) (layer "F.Cu") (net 6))
 (segment (start 161.43 86.47) (end 163.81 84.09) (width 0.2) (layer "F.Cu") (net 6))
 (segment (start 145.64 84.76) (end 147.61 82.79) (width 0.2) (layer "F.Cu") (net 6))
 (segment (start 148.52 90.48) (end 148.28 90.72) (width 0.2) (layer "F.Cu") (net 6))
 (segment (start 147.61 82.79) (end 155.16 82.79) (width 0.2) (layer "F.Cu") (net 6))
 (segment (start 148.28 90.72) (end 148.28 91.57) (width 0.2) (layer "F.Cu") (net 6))
 (segment (start 148.52 85.32) (end 148.52 90.48) (width 0.2) (layer "F.Cu") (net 6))
 (via (at 142.16 101.13) (size 0.6) (drill 0.3) (layers "F.Cu" "B.Cu") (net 6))
 (via (at 144.19 98.18) (size 0.6) (drill 0.3) (layers "F.Cu" "B.Cu") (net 6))
 (segment (start 142.16 100.21) (end 144.19 98.18) (width 0.2) (layer "B.Cu") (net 6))
 (segment (start 142.16 101.13) (end 142.16 100.21) (width 0.2) (layer "B.Cu") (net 6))
 (segment (start 147.075 101.107514) (end 147.075 101.75) (width 0.2) (layer "F.Cu") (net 5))
 (segment (start 144.61 101.22) (end 144.05 101.22) (width 0.2) (layer "F.Cu") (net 5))
 (segment (start 147.180351 101.002163) (end 147.075 101.107514) (width 0.2) (layer "F.Cu") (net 5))
 (segment (start 144.77 101.38) (end 144.61 101.22) (width 0.2) (layer "F.Cu") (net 5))
 (via (at 147.180351 101.002163) (size 0.6) (drill 0.3) (layers "F.Cu" "B.Cu") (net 5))
 (via (at 144.77 101.38) (size 0.6) (drill 0.3) (layers "F.Cu" "B.Cu") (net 5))
 (segment (start 144.77 101.38) (end 144.92 101.53) (width 0.2) (layer "B.Cu") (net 5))
 (segment (start 146.652514 101.53) (end 147.180351 101.002163) (width 0.2) (layer "B.Cu") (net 5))
 (segment (start 144.92 101.53) (end 146.652514 101.53) (width 0.2) (layer "B.Cu") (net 5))
 (segment (start 143.005 105.12) (end 142.74 105.12) (width 0.2) (layer "F.Cu") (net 9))
 (segment (start 146.525 101.6) (end 143.005 105.12) (width 0.2) (layer "F.Cu") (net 9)))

